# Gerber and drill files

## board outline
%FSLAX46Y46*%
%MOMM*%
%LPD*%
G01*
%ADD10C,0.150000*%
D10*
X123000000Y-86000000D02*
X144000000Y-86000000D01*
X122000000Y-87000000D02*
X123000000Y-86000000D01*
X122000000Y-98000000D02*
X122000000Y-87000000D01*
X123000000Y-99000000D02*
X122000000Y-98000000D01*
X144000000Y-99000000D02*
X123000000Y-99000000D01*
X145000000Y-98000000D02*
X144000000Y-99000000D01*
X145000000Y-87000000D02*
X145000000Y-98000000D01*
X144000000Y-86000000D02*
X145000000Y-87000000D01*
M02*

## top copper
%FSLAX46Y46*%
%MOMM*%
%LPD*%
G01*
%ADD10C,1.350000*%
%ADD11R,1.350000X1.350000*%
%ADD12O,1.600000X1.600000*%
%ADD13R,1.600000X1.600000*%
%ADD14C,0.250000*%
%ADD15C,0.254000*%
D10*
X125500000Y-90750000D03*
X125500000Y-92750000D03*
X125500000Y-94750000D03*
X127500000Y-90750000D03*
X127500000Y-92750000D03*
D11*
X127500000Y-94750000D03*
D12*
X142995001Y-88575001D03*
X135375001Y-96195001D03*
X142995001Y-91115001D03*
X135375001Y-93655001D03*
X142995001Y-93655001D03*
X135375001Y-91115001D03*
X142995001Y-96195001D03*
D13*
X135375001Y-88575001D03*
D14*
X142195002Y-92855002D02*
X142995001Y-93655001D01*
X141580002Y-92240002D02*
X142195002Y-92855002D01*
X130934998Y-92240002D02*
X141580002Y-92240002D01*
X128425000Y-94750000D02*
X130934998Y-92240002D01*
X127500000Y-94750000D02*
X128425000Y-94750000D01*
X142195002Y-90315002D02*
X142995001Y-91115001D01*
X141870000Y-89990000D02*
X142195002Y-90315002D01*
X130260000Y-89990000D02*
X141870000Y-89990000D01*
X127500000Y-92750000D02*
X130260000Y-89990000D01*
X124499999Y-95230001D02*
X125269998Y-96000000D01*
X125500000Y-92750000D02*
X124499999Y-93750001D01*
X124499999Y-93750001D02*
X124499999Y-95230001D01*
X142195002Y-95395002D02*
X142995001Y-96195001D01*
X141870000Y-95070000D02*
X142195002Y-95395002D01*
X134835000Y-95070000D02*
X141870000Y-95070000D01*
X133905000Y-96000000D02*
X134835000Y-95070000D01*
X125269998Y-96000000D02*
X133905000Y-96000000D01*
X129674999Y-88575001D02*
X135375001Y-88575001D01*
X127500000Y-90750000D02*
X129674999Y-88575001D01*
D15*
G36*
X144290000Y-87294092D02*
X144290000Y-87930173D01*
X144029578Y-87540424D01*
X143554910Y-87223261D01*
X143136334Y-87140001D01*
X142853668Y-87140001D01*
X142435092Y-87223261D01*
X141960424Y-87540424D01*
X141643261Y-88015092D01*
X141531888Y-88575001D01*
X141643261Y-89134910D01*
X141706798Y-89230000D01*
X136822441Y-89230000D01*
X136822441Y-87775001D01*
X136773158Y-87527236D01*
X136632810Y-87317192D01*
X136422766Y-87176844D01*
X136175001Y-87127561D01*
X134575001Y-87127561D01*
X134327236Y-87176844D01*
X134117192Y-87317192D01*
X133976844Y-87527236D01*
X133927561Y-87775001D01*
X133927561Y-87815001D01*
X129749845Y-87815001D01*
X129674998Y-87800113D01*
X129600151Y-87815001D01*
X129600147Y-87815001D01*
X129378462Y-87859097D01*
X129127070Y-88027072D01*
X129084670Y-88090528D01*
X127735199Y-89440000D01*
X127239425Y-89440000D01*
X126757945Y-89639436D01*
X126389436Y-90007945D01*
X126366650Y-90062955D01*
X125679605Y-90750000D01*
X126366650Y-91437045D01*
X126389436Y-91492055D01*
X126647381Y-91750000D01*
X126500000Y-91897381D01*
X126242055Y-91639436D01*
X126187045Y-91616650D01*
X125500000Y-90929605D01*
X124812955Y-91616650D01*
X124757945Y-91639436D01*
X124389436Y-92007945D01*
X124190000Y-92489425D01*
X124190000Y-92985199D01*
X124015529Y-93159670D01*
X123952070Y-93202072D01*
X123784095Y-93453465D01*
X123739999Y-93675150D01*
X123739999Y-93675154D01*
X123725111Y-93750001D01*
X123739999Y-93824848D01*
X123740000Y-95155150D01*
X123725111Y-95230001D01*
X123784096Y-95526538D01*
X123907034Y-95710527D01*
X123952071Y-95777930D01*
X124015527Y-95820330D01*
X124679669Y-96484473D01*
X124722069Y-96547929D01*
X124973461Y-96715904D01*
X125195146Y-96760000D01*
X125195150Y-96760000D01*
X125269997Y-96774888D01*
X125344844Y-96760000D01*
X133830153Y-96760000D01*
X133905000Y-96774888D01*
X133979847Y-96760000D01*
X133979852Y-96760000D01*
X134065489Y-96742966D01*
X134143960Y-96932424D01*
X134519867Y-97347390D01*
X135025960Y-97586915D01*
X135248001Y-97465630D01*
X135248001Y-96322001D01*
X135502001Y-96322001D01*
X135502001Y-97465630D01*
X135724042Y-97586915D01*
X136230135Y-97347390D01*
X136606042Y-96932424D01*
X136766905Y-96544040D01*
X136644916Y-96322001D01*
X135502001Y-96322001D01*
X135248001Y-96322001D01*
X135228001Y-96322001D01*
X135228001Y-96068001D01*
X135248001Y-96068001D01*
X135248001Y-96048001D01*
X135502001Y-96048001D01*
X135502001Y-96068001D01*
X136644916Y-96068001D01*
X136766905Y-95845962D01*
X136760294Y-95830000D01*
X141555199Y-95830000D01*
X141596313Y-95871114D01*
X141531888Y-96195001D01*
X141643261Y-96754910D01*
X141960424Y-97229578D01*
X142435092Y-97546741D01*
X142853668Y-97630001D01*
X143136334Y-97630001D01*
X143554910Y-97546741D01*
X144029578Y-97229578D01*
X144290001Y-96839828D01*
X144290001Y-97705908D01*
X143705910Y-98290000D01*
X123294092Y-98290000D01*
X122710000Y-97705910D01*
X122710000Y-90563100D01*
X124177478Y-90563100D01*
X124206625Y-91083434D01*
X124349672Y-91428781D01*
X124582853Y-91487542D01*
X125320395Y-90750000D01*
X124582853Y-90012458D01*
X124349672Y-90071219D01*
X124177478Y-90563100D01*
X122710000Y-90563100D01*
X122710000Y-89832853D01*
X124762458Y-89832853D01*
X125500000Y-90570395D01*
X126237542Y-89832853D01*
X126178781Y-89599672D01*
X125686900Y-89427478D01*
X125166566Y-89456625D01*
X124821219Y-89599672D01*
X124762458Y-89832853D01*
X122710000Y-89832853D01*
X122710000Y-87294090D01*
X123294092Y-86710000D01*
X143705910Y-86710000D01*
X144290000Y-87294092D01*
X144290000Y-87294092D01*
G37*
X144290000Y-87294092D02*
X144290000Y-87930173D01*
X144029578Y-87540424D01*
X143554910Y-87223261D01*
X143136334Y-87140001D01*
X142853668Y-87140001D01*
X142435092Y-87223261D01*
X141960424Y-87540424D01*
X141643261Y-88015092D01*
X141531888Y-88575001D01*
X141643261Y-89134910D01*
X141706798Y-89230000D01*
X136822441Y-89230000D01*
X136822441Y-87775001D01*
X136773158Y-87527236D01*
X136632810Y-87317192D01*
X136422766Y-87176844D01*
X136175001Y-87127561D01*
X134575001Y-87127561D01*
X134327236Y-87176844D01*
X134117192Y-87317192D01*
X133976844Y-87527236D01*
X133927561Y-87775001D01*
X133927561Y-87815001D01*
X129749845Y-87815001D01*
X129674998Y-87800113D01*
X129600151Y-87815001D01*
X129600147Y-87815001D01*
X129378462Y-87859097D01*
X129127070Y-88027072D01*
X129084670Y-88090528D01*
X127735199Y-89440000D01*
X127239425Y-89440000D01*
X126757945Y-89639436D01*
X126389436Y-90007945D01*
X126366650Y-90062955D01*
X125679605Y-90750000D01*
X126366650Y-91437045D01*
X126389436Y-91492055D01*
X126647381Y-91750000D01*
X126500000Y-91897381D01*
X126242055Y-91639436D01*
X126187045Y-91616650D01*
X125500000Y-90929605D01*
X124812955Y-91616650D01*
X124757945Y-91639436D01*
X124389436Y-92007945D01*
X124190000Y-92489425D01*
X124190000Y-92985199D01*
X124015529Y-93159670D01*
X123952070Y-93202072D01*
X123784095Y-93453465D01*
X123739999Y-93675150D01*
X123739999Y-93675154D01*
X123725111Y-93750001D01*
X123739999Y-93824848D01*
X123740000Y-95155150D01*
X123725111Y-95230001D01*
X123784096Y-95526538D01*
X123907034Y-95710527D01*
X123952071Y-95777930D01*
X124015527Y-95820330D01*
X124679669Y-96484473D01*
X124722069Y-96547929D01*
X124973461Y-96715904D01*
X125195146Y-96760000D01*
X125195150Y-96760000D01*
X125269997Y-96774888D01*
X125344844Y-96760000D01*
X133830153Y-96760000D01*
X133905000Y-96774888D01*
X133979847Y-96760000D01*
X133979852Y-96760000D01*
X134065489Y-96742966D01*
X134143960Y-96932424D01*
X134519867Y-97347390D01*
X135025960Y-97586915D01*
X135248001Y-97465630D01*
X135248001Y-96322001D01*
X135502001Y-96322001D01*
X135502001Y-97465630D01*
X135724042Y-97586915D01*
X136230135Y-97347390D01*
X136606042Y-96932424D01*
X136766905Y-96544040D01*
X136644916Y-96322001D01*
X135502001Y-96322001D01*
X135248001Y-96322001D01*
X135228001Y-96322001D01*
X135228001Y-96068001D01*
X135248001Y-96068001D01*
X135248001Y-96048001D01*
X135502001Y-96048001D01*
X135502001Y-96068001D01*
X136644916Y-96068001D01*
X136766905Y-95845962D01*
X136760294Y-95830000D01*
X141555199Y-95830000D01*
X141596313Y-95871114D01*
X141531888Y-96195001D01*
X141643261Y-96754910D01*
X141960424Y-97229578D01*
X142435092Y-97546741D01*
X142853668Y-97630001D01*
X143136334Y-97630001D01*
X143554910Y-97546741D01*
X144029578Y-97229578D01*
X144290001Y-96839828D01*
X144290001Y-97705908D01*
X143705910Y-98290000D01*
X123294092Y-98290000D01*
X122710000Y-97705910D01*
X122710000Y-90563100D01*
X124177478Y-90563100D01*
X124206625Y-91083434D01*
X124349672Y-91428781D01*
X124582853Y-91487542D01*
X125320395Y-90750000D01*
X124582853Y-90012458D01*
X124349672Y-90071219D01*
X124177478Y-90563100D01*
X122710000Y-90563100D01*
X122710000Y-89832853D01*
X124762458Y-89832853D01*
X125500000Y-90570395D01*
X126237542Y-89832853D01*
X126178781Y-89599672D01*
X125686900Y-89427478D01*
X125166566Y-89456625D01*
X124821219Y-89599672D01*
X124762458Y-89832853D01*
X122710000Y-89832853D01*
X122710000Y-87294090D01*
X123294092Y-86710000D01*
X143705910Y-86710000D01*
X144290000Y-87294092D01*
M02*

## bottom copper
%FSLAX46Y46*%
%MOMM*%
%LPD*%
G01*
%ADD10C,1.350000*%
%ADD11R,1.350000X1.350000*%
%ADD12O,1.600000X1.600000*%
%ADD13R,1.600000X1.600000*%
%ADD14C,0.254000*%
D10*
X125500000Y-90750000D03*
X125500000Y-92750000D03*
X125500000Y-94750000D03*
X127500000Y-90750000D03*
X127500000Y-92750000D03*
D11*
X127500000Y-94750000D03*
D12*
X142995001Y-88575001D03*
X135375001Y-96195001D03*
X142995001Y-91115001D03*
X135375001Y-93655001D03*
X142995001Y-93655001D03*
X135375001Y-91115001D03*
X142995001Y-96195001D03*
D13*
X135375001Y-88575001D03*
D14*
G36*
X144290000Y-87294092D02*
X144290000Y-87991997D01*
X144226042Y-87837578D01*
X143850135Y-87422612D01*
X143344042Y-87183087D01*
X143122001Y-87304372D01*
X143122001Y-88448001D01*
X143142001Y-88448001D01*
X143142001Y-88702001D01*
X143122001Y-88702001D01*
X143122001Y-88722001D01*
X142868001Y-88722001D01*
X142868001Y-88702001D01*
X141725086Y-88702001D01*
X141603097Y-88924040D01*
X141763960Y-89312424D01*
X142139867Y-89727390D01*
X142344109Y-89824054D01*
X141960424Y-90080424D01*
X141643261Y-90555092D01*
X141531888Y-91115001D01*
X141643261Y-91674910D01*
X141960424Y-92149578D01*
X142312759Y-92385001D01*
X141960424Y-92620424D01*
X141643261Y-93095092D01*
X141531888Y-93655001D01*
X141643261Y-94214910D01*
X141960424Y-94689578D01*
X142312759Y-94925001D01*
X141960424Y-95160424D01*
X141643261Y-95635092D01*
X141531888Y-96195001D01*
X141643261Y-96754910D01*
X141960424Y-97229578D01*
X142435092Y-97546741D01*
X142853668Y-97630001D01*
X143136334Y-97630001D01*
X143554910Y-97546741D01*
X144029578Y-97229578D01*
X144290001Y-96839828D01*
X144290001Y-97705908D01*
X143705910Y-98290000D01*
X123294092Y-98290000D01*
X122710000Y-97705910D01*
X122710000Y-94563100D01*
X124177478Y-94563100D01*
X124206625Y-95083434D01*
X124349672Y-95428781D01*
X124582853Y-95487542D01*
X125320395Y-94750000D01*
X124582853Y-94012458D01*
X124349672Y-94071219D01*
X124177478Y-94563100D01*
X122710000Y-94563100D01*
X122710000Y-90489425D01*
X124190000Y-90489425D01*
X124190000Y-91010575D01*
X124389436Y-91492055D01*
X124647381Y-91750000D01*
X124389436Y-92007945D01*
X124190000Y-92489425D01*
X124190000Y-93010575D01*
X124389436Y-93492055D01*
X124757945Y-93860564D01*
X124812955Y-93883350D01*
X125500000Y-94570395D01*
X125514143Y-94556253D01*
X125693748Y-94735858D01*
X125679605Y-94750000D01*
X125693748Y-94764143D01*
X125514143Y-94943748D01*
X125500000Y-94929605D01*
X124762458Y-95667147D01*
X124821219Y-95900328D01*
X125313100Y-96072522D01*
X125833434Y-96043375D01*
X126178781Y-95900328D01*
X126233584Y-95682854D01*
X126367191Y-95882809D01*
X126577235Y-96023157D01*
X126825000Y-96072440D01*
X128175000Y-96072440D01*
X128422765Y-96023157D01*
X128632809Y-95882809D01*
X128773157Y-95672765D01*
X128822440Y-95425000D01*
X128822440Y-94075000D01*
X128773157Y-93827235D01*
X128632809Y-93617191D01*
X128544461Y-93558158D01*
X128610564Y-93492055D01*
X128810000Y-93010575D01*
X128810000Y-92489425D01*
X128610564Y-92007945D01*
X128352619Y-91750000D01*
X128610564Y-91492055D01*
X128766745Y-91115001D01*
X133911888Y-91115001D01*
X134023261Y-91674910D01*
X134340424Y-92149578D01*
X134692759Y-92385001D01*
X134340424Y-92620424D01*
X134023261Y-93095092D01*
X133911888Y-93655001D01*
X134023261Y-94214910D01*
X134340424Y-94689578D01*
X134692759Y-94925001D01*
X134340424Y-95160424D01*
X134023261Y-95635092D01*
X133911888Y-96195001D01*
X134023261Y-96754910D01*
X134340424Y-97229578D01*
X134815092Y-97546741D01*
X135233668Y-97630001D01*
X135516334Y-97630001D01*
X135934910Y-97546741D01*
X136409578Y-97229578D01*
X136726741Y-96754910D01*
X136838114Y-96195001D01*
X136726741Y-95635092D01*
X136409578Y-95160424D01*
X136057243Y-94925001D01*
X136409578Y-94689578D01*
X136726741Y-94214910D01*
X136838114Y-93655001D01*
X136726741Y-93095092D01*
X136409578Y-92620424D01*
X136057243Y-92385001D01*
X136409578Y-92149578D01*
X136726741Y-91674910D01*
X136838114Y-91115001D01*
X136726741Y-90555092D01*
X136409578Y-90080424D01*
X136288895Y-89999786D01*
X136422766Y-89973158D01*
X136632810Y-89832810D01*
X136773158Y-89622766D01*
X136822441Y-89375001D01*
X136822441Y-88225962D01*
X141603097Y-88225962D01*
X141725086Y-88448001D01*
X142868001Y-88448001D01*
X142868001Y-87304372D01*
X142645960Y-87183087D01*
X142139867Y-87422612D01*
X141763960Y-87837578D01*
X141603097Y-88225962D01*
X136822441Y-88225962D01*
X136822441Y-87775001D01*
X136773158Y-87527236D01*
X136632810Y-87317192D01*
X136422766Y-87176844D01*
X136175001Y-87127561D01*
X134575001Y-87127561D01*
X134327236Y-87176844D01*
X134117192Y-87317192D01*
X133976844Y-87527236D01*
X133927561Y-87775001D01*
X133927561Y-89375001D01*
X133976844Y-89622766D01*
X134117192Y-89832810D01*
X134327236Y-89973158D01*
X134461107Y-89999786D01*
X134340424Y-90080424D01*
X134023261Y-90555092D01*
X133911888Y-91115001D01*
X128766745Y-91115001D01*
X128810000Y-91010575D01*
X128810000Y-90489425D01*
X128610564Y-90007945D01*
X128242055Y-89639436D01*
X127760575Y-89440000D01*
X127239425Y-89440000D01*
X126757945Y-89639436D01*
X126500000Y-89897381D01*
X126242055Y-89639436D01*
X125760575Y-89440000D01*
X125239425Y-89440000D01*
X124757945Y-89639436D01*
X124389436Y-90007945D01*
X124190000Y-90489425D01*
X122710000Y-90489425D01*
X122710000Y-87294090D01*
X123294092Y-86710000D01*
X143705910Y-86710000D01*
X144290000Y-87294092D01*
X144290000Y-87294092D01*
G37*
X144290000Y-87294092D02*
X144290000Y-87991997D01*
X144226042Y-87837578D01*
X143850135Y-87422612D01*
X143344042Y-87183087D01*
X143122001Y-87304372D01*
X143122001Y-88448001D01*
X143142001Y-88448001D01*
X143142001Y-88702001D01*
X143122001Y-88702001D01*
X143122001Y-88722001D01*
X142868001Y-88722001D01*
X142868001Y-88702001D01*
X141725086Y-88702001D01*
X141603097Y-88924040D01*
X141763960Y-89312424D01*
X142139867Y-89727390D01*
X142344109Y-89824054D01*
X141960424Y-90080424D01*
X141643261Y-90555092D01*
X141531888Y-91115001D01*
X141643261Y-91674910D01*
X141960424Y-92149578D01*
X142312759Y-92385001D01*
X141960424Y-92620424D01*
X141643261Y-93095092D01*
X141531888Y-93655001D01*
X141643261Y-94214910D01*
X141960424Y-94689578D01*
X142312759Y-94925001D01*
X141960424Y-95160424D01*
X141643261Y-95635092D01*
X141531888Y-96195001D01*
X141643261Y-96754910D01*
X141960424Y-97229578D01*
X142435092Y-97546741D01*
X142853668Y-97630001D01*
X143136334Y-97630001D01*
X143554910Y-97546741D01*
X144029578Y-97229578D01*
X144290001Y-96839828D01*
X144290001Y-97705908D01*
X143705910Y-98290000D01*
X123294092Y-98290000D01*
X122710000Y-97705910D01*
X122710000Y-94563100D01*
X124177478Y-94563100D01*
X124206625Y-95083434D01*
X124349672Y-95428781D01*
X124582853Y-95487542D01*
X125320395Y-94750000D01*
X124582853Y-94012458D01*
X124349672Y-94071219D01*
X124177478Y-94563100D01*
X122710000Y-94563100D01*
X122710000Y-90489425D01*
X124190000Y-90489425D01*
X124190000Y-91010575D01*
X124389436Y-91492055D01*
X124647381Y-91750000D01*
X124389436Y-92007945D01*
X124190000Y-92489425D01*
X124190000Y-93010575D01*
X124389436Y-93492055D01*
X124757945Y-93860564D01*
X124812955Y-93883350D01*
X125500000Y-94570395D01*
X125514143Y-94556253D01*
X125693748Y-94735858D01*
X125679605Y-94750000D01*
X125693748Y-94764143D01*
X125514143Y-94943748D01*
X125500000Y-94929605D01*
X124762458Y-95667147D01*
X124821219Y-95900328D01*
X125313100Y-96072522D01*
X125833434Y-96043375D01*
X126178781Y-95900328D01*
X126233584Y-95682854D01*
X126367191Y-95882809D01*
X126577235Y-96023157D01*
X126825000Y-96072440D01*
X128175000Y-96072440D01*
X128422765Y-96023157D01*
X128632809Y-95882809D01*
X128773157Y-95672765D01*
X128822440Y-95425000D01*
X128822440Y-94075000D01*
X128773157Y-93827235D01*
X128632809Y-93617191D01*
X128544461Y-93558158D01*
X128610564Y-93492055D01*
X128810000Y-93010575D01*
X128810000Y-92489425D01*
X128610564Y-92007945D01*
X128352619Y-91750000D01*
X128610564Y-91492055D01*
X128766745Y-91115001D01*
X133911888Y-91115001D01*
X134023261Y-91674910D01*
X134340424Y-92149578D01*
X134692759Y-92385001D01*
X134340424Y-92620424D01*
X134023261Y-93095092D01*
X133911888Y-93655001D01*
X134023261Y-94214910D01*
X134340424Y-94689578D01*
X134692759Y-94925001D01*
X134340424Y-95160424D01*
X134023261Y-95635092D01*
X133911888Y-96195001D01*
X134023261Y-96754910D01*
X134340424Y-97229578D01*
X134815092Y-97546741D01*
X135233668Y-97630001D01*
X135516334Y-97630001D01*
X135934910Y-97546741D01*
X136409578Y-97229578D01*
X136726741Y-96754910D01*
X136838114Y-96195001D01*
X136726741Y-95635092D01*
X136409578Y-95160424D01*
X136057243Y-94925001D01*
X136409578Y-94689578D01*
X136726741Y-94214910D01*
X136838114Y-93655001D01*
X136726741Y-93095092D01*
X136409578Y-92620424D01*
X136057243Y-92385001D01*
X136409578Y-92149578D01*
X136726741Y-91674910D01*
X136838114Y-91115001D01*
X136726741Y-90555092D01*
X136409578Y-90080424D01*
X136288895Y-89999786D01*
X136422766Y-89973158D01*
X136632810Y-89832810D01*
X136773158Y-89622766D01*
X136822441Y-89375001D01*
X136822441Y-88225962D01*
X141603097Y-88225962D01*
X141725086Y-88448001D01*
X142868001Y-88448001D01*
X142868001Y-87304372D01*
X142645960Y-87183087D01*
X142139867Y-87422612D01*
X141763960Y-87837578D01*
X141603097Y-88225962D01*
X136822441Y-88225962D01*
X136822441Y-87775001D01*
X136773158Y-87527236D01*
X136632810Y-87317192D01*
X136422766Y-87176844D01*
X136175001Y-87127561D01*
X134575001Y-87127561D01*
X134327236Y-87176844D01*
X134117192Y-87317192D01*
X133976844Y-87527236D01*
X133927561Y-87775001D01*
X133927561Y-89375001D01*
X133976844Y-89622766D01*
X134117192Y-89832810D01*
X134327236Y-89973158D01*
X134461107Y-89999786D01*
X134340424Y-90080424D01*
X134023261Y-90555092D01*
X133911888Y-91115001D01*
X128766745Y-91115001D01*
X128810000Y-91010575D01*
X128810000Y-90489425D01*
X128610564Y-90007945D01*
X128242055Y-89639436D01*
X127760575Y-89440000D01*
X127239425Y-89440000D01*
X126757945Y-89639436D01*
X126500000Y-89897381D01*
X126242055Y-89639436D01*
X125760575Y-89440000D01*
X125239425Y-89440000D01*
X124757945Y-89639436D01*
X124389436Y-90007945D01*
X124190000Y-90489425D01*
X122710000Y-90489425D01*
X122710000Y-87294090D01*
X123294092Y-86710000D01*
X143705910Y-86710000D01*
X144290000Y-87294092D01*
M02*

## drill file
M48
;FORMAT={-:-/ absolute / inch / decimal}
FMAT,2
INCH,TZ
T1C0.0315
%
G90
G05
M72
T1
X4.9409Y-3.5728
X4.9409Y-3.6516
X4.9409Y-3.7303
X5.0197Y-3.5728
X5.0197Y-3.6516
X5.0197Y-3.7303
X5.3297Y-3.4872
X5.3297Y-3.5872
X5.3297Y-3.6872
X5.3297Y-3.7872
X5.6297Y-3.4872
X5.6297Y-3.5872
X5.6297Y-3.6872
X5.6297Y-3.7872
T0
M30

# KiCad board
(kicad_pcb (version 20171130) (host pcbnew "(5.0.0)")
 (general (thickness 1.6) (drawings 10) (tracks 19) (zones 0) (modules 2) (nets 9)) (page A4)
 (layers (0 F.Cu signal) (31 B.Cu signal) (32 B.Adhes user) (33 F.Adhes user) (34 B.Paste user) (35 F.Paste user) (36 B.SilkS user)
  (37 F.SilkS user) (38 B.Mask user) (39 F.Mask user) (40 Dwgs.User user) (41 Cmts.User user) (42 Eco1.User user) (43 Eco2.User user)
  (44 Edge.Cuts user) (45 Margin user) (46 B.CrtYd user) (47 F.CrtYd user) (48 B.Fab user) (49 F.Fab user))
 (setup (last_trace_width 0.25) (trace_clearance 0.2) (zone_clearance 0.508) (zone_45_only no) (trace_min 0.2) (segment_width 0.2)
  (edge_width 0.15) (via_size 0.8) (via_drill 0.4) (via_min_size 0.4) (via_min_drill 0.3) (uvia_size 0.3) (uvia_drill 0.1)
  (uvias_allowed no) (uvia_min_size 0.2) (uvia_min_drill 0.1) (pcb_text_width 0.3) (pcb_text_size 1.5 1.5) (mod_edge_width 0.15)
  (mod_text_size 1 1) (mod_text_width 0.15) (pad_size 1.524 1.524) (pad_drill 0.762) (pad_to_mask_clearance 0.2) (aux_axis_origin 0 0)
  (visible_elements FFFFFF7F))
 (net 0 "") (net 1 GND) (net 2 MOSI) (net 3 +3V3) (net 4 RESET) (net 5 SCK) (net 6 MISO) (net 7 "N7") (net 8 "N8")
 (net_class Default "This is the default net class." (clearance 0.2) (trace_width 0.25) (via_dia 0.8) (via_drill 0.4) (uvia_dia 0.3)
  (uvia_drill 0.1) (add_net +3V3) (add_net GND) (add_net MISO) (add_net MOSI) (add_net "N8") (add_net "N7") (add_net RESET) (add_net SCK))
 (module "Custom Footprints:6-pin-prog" (layer F.Cu) (at 127.5 94.75 90)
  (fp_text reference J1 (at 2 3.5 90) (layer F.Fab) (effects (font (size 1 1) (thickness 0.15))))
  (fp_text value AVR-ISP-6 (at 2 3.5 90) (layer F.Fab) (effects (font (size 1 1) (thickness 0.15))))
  (pad 6 thru_hole circle (at 4 -2 90) (size 1.35 1.35) (drill 0.8) (layers *.Cu *.Mask) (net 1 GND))
  (pad 4 thru_hole circle (at 2 -2 90) (size 1.35 1.35) (drill 0.8) (layers *.Cu *.Mask) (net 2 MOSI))
  (pad 2 thru_hole circle (at 0 -2 90) (size 1.35 1.35) (drill 0.8) (layers *.Cu *.Mask) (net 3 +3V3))
  (pad 5 thru_hole circle (at 4 0 90) (size 1.35 1.35) (drill 0.8) (layers *.Cu *.Mask) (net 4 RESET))
  (pad 3 thru_hole circle (at 2 0 90) (size 1.35 1.35) (drill 0.8) (layers *.Cu *.Mask) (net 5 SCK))
  (pad 1 thru_hole rect (at 0 0 90) (size 1.35 1.35) (drill 0.8) (layers *.Cu *.Mask) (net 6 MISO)))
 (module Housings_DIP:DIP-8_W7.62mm (layer F.Cu) (at 135.375001 88.575001)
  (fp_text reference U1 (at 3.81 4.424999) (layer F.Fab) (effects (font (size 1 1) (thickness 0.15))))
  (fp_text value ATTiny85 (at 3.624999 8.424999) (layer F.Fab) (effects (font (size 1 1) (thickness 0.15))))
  (pad 8 thru_hole oval (at 7.62 0) (size 1.6 1.6) (drill 0.8) (layers *.Cu *.Mask) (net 3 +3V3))
  (pad 4 thru_hole oval (at 0 7.62) (size 1.6 1.6) (drill 0.8) (layers *.Cu *.Mask) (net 1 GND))
  (pad 7 thru_hole oval (at 7.62 2.54) (size 1.6 1.6) (drill 0.8) (layers *.Cu *.Mask) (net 5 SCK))
  (pad 3 thru_hole oval (at 0 5.08) (size 1.6 1.6) (drill 0.8) (layers *.Cu *.Mask) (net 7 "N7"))
  (pad 6 thru_hole oval (at 7.62 5.08) (size 1.6 1.6) (drill 0.8) (layers *.Cu *.Mask) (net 6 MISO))
  (pad 2 thru_hole oval (at 0 2.54) (size 1.6 1.6) (drill 0.8) (layers *.Cu *.Mask) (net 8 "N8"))
  (pad 5 thru_hole oval (at 7.62 7.62) (size 1.6 1.6) (drill 0.8) (layers *.Cu *.Mask) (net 2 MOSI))
  (pad 1 thru_hole rect (at 0 0) (size 1.6 1.6) (drill 0.8) (layers *.Cu *.Mask) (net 4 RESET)))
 (gr_line (start 123 86) (end 144 86) (layer Edge.Cuts) (width 0.15))
 (gr_line (start 122 87) (end 123 86) (layer Edge.Cuts) (width 0.15))
 (gr_line (start 122 98) (end 122 87) (layer Edge.Cuts) (width 0.15))
 (gr_line (start 123 99) (end 122 98) (layer Edge.Cuts) (width 0.15))
 (gr_line (start 144 99) (end 123 99) (layer Edge.Cuts) (width 0.15))
 (gr_line (start 145 98) (end 144 99) (layer Edge.Cuts) (width 0.15))
 (gr_line (start 145 87) (end 145 98) (layer Edge.Cuts) (width 0.15))
 (gr_line (start 144 86) (end 145 87) (layer Edge.Cuts) (width 0.15))
 (segment (start 142.195002 92.855002) (end 142.995001 93.655001) (width 0.25) (layer F.Cu) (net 6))
 (segment (start 141.580002 92.240002) (end 142.195002 92.855002) (width 0.25) (layer F.Cu) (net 6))
 (segment (start 130.934998 92.240002) (end 141.580002 92.240002) (width 0.25) (layer F.Cu) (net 6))
 (segment (start 128.425 94.75) (end 130.934998 92.240002) (width 0.25) (layer F.Cu) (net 6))
 (segment (start 127.5 94.75) (end 128.425 94.75) (width 0.25) (layer F.Cu) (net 6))
 (segment (start 142.195002 90.315002) (end 142.995001 91.115001) (width 0.25) (layer F.Cu) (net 5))
 (segment (start 141.87 89.99) (end 142.195002 90.315002) (width 0.25) (layer F.Cu) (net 5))
 (segment (start 130.26 89.99) (end 141.87 89.99) (width 0.25) (layer F.Cu) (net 5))
 (segment (start 127.5 92.75) (end 130.26 89.99) (width 0.25) (layer F.Cu) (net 5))
 (segment (start 124.499999 95.230001) (end 125.269998 96) (width 0.25) (layer F.Cu) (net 2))
 (segment (start 125.5 92.75) (end 124.499999 93.750001) (width 0.25) (layer F.Cu) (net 2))
 (segment (start 124.499999 93.750001) (end 124.499999 95.230001) (width 0.25) (layer F.Cu) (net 2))
 (segment (start 142.195002 95.395002) (end 142.995001 96.195001) (width 0.25) (layer F.Cu) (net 2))
 (segment (start 141.87 95.07) (end 142.195002 95.395002) (width 0.25) (layer F.Cu) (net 2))
 (segment (start 134.835 95.07) (end 141.87 95.07) (width 0.25) (layer F.Cu) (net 2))
 (segment (start 133.905 96) (end 134.835 95.07) (width 0.25) (layer F.Cu) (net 2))
 (segment (start 125.269998 96) (end 133.905 96) (width 0.25) (layer F.Cu) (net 2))
 (segment (start 129.674999 88.575001) (end 135.375001 88.575001) (width 0.25) (layer F.Cu) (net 4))
 (segment (start 127.5 90.75) (end 129.674999 88.575001) (width 0.25) (layer F.Cu) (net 4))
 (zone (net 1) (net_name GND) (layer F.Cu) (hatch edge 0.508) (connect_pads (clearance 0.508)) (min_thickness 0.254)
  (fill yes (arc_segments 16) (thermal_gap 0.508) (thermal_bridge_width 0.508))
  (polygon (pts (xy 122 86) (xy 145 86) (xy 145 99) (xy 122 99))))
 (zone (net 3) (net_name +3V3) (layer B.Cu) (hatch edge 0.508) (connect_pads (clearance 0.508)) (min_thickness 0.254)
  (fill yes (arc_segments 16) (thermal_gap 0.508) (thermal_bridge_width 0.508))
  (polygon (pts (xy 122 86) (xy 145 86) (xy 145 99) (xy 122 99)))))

